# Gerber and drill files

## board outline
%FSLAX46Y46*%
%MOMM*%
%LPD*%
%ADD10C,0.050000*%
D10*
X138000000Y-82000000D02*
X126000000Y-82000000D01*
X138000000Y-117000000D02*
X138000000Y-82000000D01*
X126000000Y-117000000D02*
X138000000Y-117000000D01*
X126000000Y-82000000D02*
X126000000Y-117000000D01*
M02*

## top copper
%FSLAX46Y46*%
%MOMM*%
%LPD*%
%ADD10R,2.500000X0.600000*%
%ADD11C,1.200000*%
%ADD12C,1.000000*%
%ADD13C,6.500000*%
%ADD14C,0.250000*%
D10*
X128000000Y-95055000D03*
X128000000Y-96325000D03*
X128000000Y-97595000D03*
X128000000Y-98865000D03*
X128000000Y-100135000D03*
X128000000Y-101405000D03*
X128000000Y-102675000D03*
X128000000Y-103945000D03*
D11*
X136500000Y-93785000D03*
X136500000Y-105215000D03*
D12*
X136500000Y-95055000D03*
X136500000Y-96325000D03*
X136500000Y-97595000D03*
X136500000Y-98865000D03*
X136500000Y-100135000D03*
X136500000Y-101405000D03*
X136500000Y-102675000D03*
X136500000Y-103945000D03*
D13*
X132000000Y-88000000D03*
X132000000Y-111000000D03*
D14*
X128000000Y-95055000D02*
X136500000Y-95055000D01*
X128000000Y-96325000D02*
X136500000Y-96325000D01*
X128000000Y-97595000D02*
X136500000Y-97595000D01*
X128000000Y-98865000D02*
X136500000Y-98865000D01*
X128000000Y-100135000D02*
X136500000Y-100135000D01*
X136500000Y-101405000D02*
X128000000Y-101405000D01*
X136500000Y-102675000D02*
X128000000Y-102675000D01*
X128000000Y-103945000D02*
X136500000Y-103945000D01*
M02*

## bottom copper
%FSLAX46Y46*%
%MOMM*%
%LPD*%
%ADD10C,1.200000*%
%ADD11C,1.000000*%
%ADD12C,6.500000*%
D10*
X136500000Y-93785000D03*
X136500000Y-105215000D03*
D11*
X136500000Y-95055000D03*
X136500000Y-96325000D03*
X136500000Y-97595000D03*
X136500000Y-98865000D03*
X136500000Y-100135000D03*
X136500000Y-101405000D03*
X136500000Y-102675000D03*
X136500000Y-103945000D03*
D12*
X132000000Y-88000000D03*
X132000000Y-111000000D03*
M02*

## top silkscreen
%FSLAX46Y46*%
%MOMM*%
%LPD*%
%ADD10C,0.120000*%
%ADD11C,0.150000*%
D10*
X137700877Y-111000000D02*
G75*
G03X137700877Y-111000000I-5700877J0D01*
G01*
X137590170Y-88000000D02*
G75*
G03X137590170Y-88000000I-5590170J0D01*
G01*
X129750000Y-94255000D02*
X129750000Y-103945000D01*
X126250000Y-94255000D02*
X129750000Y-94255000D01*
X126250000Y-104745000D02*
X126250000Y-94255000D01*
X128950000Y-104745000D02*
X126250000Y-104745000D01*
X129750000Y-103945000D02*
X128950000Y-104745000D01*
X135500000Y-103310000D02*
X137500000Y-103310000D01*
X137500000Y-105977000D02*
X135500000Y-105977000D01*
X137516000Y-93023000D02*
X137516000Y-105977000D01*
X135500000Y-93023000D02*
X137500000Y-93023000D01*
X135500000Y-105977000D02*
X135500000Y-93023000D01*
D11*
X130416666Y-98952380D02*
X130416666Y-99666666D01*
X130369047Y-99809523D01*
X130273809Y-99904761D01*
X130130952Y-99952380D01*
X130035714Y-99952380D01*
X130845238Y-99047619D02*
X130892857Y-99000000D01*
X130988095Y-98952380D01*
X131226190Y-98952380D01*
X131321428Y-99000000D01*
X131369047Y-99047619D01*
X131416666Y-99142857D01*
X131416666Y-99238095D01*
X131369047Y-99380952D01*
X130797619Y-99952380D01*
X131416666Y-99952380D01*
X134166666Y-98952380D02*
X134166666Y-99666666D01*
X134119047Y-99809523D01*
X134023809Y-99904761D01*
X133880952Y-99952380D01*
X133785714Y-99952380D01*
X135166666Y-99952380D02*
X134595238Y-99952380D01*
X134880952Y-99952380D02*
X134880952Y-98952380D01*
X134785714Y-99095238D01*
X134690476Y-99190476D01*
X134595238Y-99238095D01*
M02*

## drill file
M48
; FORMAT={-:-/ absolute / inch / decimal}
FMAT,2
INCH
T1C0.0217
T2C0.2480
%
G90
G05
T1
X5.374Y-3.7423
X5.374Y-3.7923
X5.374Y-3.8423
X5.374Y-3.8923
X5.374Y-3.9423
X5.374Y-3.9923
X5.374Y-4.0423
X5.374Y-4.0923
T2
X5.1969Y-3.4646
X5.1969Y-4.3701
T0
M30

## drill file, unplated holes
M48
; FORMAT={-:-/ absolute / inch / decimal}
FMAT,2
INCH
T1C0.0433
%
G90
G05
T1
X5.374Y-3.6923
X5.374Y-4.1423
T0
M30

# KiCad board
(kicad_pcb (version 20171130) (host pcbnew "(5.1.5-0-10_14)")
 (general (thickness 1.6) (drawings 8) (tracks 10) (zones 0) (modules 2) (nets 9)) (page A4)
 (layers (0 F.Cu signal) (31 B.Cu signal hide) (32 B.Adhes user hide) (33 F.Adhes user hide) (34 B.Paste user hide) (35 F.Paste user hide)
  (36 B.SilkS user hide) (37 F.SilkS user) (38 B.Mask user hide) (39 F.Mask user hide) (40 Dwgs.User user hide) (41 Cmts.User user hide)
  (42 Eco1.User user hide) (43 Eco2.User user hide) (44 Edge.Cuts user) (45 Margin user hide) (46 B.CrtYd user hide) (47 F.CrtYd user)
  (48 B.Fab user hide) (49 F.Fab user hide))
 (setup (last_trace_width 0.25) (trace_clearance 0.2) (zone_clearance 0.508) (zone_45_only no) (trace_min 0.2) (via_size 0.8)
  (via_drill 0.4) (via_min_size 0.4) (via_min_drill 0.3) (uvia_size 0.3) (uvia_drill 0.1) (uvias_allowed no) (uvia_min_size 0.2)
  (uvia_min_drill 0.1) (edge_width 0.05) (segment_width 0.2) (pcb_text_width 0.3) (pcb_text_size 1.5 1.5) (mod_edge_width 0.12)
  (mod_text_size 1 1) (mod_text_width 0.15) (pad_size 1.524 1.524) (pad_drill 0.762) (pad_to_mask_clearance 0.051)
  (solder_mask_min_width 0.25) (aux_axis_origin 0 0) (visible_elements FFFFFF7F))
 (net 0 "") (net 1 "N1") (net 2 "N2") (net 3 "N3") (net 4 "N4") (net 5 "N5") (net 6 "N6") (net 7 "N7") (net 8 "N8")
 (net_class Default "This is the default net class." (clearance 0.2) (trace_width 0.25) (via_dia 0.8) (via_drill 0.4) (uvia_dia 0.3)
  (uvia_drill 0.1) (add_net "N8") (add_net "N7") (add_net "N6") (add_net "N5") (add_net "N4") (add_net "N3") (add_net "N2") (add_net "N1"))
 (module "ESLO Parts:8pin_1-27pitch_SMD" (layer F.Cu) (at 128 99.5 90)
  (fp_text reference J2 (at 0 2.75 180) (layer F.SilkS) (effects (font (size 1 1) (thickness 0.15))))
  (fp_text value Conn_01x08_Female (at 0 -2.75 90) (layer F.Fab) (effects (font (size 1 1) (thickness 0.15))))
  (fp_line (start 5.245 1.75) (end -4.445 1.75) (layer F.SilkS) (width 0.12))
  (fp_line (start 5.245 -1.75) (end 5.245 1.75) (layer F.SilkS) (width 0.12))
  (fp_line (start -5.245 -1.75) (end 5.245 -1.75) (layer F.SilkS) (width 0.12))
  (fp_line (start -5.245 0.95) (end -5.245 -1.75) (layer F.SilkS) (width 0.12))
  (fp_line (start -4.445 1.75) (end -5.245 0.95) (layer F.SilkS) (width 0.12))
  (pad 8 smd rect (at 4.445 0 90) (size 0.6 2.5) (layers F.Cu F.Paste F.Mask) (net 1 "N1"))
  (pad 7 smd rect (at 3.175 0 90) (size 0.6 2.5) (layers F.Cu F.Paste F.Mask) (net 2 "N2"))
  (pad 6 smd rect (at 1.905 0 90) (size 0.6 2.5) (layers F.Cu F.Paste F.Mask) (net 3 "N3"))
  (pad 5 smd rect (at 0.635 0 90) (size 0.6 2.5) (layers F.Cu F.Paste F.Mask) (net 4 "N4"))
  (pad 4 smd rect (at -0.635 0 90) (size 0.6 2.5) (layers F.Cu F.Paste F.Mask) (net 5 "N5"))
  (pad 3 smd rect (at -1.905 0 90) (size 0.6 2.5) (layers F.Cu F.Paste F.Mask) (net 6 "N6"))
  (pad 2 smd rect (at -3.175 0 90) (size 0.6 2.5) (layers F.Cu F.Paste F.Mask) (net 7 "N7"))
  (pad 1 smd rect (at -4.445 0 90) (size 0.6 2.5) (layers F.Cu F.Paste F.Mask) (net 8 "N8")))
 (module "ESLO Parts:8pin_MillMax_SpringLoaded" (layer F.Cu) (at 136.5 99.5 90)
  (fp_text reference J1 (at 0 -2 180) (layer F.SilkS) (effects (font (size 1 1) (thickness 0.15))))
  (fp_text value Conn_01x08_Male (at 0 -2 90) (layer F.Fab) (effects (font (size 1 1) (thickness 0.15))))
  (fp_line (start -3.81 -1) (end -3.81 1) (layer F.SilkS) (width 0.12))
  (fp_line (start -6.477 1) (end -6.477 -1) (layer F.SilkS) (width 0.12))
  (fp_line (start 6.477 1.016) (end -6.477 1.016) (layer F.SilkS) (width 0.12))
  (fp_line (start 6.477 -1) (end 6.477 1) (layer F.SilkS) (width 0.12))
  (fp_line (start -6.477 -1) (end 6.477 -1) (layer F.SilkS) (width 0.12))
  (pad "" np_thru_hole circle (at 5.715 0 90) (size 1.2 1.2) (drill 1.1) (layers *.Cu *.Mask))
  (pad "" np_thru_hole circle (at -5.715 0 90) (size 1.2 1.2) (drill 1.1) (layers *.Cu *.Mask))
  (pad 8 thru_hole circle (at 4.445 0 90) (size 1 1) (drill 0.55) (layers *.Cu *.Mask) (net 1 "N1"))
  (pad 7 thru_hole circle (at 3.175 0 90) (size 1 1) (drill 0.55) (layers *.Cu *.Mask) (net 2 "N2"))
  (pad 6 thru_hole circle (at 1.905 0 90) (size 1 1) (drill 0.55) (layers *.Cu *.Mask) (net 3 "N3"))
  (pad 5 thru_hole circle (at 0.635 0 90) (size 1 1) (drill 0.55) (layers *.Cu *.Mask) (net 4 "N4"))
  (pad 4 thru_hole circle (at -0.635 0 90) (size 1 1) (drill 0.55) (layers *.Cu *.Mask) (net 5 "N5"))
  (pad 3 thru_hole circle (at -1.905 0 90) (size 1 1) (drill 0.55) (layers *.Cu *.Mask) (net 6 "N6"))
  (pad 2 thru_hole circle (at -3.175 0 90) (size 1 1) (drill 0.55) (layers *.Cu *.Mask) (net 7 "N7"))
  (pad 1 thru_hole circle (at -4.445 0 90) (size 1 1) (drill 0.55) (layers *.Cu *.Mask) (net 8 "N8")))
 (gr_circle (center 132 111) (end 136.5 114.5) (layer F.SilkS) (width 0.12))
 (gr_circle (center 132 88) (end 137 90.5) (layer F.SilkS) (width 0.12))
 (gr_line (start 138 82) (end 126 82) (layer Edge.Cuts) (width 0.05))
 (gr_line (start 138 117) (end 138 82) (layer Edge.Cuts) (width 0.05))
 (gr_line (start 126 117) (end 138 117) (layer Edge.Cuts) (width 0.05))
 (gr_line (start 126 82) (end 126 117) (layer Edge.Cuts) (width 0.05))
 (via (at 132 88) (size 6.5) (drill 6.3) (layers F.Cu B.Cu) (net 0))
 (via (at 132 111) (size 6.5) (drill 6.3) (layers F.Cu B.Cu) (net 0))
 (segment (start 128 95.055) (end 136.5 95.055) (width 0.25) (layer F.Cu) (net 1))
 (segment (start 128 96.325) (end 136.5 96.325) (width 0.25) (layer F.Cu) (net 2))
 (segment (start 128 97.595) (end 136.5 97.595) (width 0.25) (layer F.Cu) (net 3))
 (segment (start 128 98.865) (end 136.5 98.865) (width 0.25) (layer F.Cu) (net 4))
 (segment (start 128 100.135) (end 136.5 100.135) (width 0.25) (layer F.Cu) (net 5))
 (segment (start 136.5 101.405) (end 128 101.405) (width 0.25) (layer F.Cu) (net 6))
 (segment (start 136.5 102.675) (end 128 102.675) (width 0.25) (layer F.Cu) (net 7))
 (segment (start 128 103.945) (end 136.5 103.945) (width 0.25) (layer F.Cu) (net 8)))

